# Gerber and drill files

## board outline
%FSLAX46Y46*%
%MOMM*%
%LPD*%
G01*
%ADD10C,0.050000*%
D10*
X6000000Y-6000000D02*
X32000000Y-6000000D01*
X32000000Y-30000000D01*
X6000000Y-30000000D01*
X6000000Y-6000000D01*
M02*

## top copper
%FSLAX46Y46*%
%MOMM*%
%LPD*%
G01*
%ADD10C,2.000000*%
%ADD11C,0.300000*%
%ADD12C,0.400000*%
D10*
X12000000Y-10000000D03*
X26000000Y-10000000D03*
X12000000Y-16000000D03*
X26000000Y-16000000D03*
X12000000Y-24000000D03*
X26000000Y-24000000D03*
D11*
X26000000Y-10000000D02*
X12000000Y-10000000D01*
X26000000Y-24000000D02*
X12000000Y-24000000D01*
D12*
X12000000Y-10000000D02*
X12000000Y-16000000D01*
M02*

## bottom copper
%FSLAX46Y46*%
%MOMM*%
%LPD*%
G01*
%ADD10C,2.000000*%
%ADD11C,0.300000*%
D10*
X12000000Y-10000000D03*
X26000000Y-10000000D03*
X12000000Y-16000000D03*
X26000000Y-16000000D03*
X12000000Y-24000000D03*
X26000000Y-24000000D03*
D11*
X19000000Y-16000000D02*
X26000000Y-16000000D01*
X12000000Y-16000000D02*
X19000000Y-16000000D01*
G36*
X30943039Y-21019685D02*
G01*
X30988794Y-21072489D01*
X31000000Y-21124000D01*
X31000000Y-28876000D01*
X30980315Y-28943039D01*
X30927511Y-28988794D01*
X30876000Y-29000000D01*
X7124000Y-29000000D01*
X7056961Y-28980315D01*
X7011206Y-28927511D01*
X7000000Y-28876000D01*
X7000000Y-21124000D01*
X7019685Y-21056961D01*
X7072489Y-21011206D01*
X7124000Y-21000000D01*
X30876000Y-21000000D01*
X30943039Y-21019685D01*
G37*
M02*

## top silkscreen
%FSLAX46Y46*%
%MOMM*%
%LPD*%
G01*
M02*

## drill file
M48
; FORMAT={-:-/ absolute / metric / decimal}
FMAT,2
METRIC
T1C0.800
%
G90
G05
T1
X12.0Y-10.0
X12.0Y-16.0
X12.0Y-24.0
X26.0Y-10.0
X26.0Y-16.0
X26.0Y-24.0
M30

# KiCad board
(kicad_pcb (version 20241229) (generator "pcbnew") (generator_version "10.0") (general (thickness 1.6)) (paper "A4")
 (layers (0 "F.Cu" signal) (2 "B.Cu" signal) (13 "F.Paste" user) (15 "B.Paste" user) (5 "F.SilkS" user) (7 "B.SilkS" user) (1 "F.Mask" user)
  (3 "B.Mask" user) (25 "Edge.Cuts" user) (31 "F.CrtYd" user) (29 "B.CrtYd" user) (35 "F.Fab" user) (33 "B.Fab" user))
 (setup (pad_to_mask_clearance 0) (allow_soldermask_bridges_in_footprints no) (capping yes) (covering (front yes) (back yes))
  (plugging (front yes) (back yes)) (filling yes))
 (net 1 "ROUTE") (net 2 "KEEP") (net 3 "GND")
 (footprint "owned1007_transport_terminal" (layer "F.Cu") (at 12 10)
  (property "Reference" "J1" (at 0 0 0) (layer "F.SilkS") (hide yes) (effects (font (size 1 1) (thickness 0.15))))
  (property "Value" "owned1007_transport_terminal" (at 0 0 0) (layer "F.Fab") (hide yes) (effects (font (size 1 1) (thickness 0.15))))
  (pad "1" thru_hole circle (at 0 0) (size 2 2) (drill 0.8) (layers "*.Cu" "*.Mask") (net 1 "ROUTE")))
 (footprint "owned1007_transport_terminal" (layer "F.Cu") (at 26 10)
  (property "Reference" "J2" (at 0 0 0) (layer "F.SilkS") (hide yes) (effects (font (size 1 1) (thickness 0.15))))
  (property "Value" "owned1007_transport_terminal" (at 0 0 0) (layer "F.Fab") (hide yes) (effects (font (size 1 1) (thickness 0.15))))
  (pad "1" thru_hole circle (at 0 0) (size 2 2) (drill 0.8) (layers "*.Cu" "*.Mask") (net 1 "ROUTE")))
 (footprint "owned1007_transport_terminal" (layer "F.Cu") (at 12 16)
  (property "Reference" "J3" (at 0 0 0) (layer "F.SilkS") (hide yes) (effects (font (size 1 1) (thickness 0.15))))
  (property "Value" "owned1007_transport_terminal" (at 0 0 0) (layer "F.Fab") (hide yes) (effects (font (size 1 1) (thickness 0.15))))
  (pad "1" thru_hole circle (at 0 0) (size 2 2) (drill 0.8) (layers "*.Cu" "*.Mask") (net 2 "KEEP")))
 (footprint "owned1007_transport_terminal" (layer "F.Cu") (at 26 16)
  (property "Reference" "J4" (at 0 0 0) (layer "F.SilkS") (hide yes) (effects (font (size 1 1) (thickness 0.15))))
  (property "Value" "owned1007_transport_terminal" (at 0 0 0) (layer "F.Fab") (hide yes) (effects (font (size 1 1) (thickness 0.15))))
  (pad "1" thru_hole circle (at 0 0) (size 2 2) (drill 0.8) (layers "*.Cu" "*.Mask") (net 2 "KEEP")))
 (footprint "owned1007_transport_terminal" (layer "F.Cu") (at 12 24)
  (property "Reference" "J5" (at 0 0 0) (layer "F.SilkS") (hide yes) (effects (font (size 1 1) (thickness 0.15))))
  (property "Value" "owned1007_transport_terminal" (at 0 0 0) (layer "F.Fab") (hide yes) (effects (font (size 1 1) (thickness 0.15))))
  (pad "1" thru_hole circle (at 0 0) (size 2 2) (drill 0.8) (layers "*.Cu" "*.Mask") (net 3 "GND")))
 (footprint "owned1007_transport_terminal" (layer "F.Cu") (at 26 24)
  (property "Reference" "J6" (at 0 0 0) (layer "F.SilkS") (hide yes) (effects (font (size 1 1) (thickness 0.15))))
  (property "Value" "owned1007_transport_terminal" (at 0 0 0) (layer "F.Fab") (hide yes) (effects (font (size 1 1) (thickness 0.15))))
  (pad "1" thru_hole circle (at 0 0) (size 2 2) (drill 0.8) (layers "*.Cu" "*.Mask") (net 3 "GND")))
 (gr_rect (start 6 6) (end 32 30) (stroke (width 0.05) (type default)) (fill none) (layer "Edge.Cuts"))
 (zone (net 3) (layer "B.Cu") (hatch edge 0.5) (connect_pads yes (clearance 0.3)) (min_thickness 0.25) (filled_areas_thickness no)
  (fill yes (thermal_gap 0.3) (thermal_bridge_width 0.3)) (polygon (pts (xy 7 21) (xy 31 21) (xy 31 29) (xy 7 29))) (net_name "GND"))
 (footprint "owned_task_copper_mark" (layer "F.Cu") (at 10 28)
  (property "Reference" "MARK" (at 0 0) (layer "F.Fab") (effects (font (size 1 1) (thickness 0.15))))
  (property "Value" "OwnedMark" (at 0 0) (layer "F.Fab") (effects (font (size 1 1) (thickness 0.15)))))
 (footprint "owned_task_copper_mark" (layer "F.Cu") (at 13 28)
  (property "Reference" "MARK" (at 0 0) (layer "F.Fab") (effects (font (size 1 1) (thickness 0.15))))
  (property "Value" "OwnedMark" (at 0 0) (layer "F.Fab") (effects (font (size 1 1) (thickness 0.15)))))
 (segment (start 26 10) (end 12 10) (width 0.3) (layer "F.Cu") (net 1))
 (segment (start 19 16) (end 26 16) (width 0.3) (layer "B.Cu") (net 2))
 (segment (start 12 16) (end 19 16) (width 0.3) (layer "B.Cu") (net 2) (locked yes))
 (segment (start 26 24) (end 12 24) (width 0.3) (layer "F.Cu") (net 3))
 (segment (start 12 10) (end 12 16) (width 0.4) (layer "F.Cu") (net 1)))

